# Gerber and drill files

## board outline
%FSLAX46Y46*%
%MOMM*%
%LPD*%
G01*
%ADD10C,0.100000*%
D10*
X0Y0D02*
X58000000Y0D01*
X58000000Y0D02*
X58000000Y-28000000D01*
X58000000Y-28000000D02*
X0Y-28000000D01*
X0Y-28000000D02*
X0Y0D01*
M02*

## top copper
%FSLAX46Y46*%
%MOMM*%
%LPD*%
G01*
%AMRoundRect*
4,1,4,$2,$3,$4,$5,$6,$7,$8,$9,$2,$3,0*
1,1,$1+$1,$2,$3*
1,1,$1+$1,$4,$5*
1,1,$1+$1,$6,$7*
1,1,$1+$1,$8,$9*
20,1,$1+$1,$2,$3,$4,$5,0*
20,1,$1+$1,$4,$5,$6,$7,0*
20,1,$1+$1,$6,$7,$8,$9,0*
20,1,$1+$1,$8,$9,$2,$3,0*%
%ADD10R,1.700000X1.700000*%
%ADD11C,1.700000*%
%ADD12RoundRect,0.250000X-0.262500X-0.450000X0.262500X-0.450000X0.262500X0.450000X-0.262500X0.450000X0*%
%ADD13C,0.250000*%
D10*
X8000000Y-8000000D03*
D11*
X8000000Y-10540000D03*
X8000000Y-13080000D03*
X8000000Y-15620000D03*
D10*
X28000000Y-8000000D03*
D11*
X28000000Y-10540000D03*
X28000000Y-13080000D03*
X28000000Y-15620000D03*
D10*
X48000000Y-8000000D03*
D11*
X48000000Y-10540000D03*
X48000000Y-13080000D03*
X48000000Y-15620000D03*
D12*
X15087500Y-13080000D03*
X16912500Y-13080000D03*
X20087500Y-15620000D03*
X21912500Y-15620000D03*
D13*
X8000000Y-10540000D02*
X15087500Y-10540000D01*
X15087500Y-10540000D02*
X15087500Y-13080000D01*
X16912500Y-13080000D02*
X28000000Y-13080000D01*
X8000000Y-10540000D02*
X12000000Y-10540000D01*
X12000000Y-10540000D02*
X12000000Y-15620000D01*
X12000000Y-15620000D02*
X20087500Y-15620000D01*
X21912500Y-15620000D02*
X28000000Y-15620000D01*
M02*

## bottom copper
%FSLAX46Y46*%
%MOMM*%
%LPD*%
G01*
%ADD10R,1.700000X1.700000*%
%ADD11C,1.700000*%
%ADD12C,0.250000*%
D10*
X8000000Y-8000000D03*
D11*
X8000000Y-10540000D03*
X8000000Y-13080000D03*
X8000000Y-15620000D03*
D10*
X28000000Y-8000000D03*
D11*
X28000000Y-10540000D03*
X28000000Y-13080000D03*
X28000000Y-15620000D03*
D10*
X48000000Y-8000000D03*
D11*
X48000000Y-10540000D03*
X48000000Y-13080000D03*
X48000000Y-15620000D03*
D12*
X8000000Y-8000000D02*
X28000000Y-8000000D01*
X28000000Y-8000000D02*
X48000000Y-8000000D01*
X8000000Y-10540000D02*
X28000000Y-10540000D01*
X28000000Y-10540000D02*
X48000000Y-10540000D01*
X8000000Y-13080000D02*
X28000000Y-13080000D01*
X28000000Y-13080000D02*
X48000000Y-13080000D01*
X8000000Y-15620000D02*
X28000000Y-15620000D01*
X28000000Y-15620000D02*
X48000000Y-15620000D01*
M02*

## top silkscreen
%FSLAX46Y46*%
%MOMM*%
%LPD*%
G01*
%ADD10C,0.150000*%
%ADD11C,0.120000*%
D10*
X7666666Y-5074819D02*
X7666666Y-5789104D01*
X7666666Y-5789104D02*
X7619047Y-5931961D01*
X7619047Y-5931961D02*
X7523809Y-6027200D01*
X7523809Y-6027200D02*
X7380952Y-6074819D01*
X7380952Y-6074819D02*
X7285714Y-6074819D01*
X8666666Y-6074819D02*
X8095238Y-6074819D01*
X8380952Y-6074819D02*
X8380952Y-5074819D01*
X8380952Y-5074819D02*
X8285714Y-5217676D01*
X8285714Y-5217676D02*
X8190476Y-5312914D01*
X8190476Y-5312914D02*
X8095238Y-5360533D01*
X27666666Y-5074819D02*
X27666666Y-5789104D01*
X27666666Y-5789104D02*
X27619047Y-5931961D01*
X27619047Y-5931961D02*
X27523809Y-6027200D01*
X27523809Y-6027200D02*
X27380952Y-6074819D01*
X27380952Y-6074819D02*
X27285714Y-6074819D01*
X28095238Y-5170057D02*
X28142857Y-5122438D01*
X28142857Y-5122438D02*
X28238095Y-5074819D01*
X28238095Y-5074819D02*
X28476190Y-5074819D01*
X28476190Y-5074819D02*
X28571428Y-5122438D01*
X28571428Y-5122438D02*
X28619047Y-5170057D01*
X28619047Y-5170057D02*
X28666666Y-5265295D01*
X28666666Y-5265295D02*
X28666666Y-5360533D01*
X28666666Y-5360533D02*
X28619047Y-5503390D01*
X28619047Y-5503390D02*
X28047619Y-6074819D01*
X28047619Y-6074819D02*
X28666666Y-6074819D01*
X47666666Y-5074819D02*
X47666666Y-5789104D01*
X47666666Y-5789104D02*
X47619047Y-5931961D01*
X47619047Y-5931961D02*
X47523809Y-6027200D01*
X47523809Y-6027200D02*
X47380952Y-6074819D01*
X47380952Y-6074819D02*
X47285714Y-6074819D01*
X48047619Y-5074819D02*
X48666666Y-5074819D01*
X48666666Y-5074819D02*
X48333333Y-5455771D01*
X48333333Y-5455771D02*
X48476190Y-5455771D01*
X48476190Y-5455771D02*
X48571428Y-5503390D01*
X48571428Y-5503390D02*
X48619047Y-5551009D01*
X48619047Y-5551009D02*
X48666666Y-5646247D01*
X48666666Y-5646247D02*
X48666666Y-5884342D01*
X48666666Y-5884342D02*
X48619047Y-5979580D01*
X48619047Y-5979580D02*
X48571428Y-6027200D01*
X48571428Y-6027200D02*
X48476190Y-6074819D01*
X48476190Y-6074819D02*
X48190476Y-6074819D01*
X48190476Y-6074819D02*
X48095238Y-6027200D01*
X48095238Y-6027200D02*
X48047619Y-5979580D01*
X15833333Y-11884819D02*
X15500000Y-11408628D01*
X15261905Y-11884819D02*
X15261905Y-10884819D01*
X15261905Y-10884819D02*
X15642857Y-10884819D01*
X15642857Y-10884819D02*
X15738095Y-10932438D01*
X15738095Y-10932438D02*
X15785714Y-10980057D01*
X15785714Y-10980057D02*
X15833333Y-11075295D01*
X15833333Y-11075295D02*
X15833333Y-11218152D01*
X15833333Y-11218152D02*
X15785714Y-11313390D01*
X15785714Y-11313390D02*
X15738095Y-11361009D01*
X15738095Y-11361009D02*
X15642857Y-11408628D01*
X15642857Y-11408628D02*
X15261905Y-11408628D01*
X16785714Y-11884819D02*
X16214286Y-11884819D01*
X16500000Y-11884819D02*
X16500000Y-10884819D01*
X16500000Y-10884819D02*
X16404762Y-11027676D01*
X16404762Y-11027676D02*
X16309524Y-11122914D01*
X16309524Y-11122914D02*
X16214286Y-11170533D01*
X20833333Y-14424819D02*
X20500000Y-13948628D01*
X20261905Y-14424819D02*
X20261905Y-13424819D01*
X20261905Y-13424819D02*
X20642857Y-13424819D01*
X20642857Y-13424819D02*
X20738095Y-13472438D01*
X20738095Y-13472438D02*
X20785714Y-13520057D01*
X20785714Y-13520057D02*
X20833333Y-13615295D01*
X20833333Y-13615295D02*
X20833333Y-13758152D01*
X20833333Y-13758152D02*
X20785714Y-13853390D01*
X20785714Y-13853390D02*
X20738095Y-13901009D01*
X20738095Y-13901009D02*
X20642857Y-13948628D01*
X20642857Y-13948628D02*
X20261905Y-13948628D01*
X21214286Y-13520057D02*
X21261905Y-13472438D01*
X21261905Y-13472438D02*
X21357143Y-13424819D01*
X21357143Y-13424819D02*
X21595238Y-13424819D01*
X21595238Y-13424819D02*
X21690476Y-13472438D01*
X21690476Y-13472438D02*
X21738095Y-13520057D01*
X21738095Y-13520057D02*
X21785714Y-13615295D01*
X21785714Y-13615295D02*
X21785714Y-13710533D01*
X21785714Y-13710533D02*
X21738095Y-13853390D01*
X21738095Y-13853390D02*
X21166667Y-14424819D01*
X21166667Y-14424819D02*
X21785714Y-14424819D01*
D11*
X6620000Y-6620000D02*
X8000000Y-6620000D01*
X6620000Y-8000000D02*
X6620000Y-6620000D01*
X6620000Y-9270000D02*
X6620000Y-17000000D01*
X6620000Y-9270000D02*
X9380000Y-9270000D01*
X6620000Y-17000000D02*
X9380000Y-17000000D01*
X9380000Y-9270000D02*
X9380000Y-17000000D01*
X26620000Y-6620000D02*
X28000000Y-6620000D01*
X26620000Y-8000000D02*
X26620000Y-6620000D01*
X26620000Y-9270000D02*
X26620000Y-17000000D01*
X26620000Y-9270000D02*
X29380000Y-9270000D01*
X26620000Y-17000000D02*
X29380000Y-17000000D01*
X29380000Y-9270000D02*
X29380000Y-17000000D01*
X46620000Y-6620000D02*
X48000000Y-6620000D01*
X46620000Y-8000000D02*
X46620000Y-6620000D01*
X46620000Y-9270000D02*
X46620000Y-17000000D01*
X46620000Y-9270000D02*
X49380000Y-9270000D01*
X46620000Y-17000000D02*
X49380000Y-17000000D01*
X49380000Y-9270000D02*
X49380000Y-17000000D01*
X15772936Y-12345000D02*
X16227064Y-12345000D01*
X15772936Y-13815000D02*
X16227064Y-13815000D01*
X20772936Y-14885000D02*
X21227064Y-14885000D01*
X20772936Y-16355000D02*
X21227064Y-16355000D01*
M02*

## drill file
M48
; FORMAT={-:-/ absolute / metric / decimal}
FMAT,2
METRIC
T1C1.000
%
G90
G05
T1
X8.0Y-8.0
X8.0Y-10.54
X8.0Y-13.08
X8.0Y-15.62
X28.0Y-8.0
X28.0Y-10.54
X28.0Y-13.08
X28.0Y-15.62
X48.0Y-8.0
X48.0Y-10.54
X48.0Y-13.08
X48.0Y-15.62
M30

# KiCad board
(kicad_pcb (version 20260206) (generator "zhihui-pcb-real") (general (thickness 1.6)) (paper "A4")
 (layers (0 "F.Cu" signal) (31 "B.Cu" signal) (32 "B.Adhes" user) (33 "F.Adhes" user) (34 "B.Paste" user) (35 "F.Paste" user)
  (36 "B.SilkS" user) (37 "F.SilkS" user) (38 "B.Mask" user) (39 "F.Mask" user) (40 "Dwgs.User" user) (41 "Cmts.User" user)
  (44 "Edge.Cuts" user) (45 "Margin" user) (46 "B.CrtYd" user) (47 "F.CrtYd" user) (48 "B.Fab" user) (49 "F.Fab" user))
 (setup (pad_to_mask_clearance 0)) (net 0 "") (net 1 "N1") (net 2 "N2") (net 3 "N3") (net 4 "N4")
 (gr_line (start 0 0) (end 58 0) (stroke (width 0.1) (type default)) (layer "Edge.Cuts"))
 (gr_line (start 58 0) (end 58 28) (stroke (width 0.1) (type default)) (layer "Edge.Cuts"))
 (gr_line (start 58 28) (end 0 28) (stroke (width 0.1) (type default)) (layer "Edge.Cuts"))
 (gr_line (start 0 28) (end 0 0) (stroke (width 0.1) (type default)) (layer "Edge.Cuts"))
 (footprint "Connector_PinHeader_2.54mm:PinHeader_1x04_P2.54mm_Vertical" (layer "F.Cu")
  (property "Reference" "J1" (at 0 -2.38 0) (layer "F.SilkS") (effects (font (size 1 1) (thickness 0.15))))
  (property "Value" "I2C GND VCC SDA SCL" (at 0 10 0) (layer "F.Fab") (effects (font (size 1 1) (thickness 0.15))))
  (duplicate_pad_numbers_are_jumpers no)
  (fp_line (start -1.38 -1.38) (end 0 -1.38) (stroke (width 0.12) (type solid)) (layer "F.SilkS"))
  (fp_line (start -1.38 0) (end -1.38 -1.38) (stroke (width 0.12) (type solid)) (layer "F.SilkS"))
  (fp_line (start -1.38 1.27) (end -1.38 9) (stroke (width 0.12) (type solid)) (layer "F.SilkS"))
  (fp_line (start -1.38 1.27) (end 1.38 1.27) (stroke (width 0.12) (type solid)) (layer "F.SilkS"))
  (fp_line (start -1.38 9) (end 1.38 9) (stroke (width 0.12) (type solid)) (layer "F.SilkS"))
  (fp_line (start 1.38 1.27) (end 1.38 9) (stroke (width 0.12) (type solid)) (layer "F.SilkS"))
  (pad "1" thru_hole rect (at 0 0) (size 1.7 1.7) (drill 1) (layers "*.Cu" "*.Mask") (remove_unused_layers no) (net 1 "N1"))
  (pad "2" thru_hole circle (at 0 2.54) (size 1.7 1.7) (drill 1) (layers "*.Cu" "*.Mask") (remove_unused_layers no) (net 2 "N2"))
  (pad "3" thru_hole circle (at 0 5.08) (size 1.7 1.7) (drill 1) (layers "*.Cu" "*.Mask") (remove_unused_layers no) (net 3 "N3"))
  (pad "4" thru_hole circle (at 0 7.62) (size 1.7 1.7) (drill 1) (layers "*.Cu" "*.Mask") (remove_unused_layers no) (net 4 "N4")) (at 8 8 0))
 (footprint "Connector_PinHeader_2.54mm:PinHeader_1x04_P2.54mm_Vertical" (layer "F.Cu")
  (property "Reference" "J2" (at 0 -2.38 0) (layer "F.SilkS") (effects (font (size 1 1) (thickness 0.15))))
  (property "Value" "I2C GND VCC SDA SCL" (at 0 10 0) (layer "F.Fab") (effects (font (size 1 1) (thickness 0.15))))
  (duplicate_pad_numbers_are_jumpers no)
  (fp_line (start -1.38 -1.38) (end 0 -1.38) (stroke (width 0.12) (type solid)) (layer "F.SilkS"))
  (fp_line (start -1.38 0) (end -1.38 -1.38) (stroke (width 0.12) (type solid)) (layer "F.SilkS"))
  (fp_line (start -1.38 1.27) (end -1.38 9) (stroke (width 0.12) (type solid)) (layer "F.SilkS"))
  (fp_line (start -1.38 1.27) (end 1.38 1.27) (stroke (width 0.12) (type solid)) (layer "F.SilkS"))
  (fp_line (start -1.38 9) (end 1.38 9) (stroke (width 0.12) (type solid)) (layer "F.SilkS"))
  (fp_line (start 1.38 1.27) (end 1.38 9) (stroke (width 0.12) (type solid)) (layer "F.SilkS"))
  (pad "1" thru_hole rect (at 0 0) (size 1.7 1.7) (drill 1) (layers "*.Cu" "*.Mask") (remove_unused_layers no) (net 1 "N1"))
  (pad "2" thru_hole circle (at 0 2.54) (size 1.7 1.7) (drill 1) (layers "*.Cu" "*.Mask") (remove_unused_layers no) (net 2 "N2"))
  (pad "3" thru_hole circle (at 0 5.08) (size 1.7 1.7) (drill 1) (layers "*.Cu" "*.Mask") (remove_unused_layers no) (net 3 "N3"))
  (pad "4" thru_hole circle (at 0 7.62) (size 1.7 1.7) (drill 1) (layers "*.Cu" "*.Mask") (remove_unused_layers no) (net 4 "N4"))
  (at 28 8 0))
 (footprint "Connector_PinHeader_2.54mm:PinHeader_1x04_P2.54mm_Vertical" (layer "F.Cu")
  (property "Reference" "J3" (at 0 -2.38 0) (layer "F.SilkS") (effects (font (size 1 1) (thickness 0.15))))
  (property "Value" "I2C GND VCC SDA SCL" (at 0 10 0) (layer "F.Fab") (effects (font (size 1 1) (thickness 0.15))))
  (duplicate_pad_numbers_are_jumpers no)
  (fp_line (start -1.38 -1.38) (end 0 -1.38) (stroke (width 0.12) (type solid)) (layer "F.SilkS"))
  (fp_line (start -1.38 0) (end -1.38 -1.38) (stroke (width 0.12) (type solid)) (layer "F.SilkS"))
  (fp_line (start -1.38 1.27) (end -1.38 9) (stroke (width 0.12) (type solid)) (layer "F.SilkS"))
  (fp_line (start -1.38 1.27) (end 1.38 1.27) (stroke (width 0.12) (type solid)) (layer "F.SilkS"))
  (fp_line (start -1.38 9) (end 1.38 9) (stroke (width 0.12) (type solid)) (layer "F.SilkS"))
  (fp_line (start 1.38 1.27) (end 1.38 9) (stroke (width 0.12) (type solid)) (layer "F.SilkS"))
  (pad "1" thru_hole rect (at 0 0) (size 1.7 1.7) (drill 1) (layers "*.Cu" "*.Mask") (remove_unused_layers no) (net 1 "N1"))
  (pad "2" thru_hole circle (at 0 2.54) (size 1.7 1.7) (drill 1) (layers "*.Cu" "*.Mask") (remove_unused_layers no) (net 2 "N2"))
  (pad "3" thru_hole circle (at 0 5.08) (size 1.7 1.7) (drill 1) (layers "*.Cu" "*.Mask") (remove_unused_layers no) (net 3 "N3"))
  (pad "4" thru_hole circle (at 0 7.62) (size 1.7 1.7) (drill 1) (layers "*.Cu" "*.Mask") (remove_unused_layers no) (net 4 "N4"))
  (at 48 8 0))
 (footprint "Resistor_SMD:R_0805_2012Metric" (layer "F.Cu")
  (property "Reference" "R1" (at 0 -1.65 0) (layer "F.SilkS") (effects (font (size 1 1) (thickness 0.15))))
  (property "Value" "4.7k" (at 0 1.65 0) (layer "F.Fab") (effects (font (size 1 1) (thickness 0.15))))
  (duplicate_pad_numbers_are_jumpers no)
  (fp_line (start -0.227064 -0.735) (end 0.227064 -0.735) (stroke (width 0.12) (type solid)) (layer "F.SilkS"))
  (fp_line (start -0.227064 0.735) (end 0.227064 0.735) (stroke (width 0.12) (type solid)) (layer "F.SilkS"))
  (pad "1" smd roundrect (at -0.9125 0) (size 1.025 1.4) (layers "F.Cu" "F.Mask" "F.Paste") (roundrect_rratio 0.243902) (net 2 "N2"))
  (pad "2" smd roundrect (at 0.9125 0) (size 1.025 1.4) (layers "F.Cu" "F.Mask" "F.Paste") (roundrect_rratio 0.243902) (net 3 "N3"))
  (at 16 13.08 0))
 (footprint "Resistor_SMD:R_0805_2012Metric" (layer "F.Cu")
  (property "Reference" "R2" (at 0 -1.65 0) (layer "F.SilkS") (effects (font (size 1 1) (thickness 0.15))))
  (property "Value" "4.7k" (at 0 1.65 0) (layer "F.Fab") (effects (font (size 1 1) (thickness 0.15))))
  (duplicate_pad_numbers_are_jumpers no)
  (fp_line (start -0.227064 -0.735) (end 0.227064 -0.735) (stroke (width 0.12) (type solid)) (layer "F.SilkS"))
  (fp_line (start -0.227064 0.735) (end 0.227064 0.735) (stroke (width 0.12) (type solid)) (layer "F.SilkS"))
  (pad "1" smd roundrect (at -0.9125 0) (size 1.025 1.4) (layers "F.Cu" "F.Mask" "F.Paste") (roundrect_rratio 0.243902) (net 2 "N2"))
  (pad "2" smd roundrect (at 0.9125 0) (size 1.025 1.4) (layers "F.Cu" "F.Mask" "F.Paste") (roundrect_rratio 0.243902) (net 4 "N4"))
  (at 21 15.62 0))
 (segment (start 8 8) (end 28 8) (width 0.25) (layer "B.Cu") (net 1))
 (segment (start 28 8) (end 48 8) (width 0.25) (layer "B.Cu") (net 1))
 (segment (start 8 10.54) (end 28 10.54) (width 0.25) (layer "B.Cu") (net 2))
 (segment (start 28 10.54) (end 48 10.54) (width 0.25) (layer "B.Cu") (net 2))
 (segment (start 8 13.08) (end 28 13.08) (width 0.25) (layer "B.Cu") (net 3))
 (segment (start 28 13.08) (end 48 13.08) (width 0.25) (layer "B.Cu") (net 3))
 (segment (start 8 15.62) (end 28 15.62) (width 0.25) (layer "B.Cu") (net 4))
 (segment (start 28 15.62) (end 48 15.62) (width 0.25) (layer "B.Cu") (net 4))
 (segment (start 8 10.54) (end 15.0875 10.54) (width 0.25) (layer "F.Cu") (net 2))
 (segment (start 15.0875 10.54) (end 15.0875 13.08) (width 0.25) (layer "F.Cu") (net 2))
 (segment (start 16.9125 13.08) (end 28 13.08) (width 0.25) (layer "F.Cu") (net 3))
 (segment (start 8 10.54) (end 12 10.54) (width 0.25) (layer "F.Cu") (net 2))
 (segment (start 12 10.54) (end 12 15.62) (width 0.25) (layer "F.Cu") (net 2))
 (segment (start 12 15.62) (end 20.0875 15.62) (width 0.25) (layer "F.Cu") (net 2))
 (segment (start 21.9125 15.62) (end 28 15.62) (width 0.25) (layer "F.Cu") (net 4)))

